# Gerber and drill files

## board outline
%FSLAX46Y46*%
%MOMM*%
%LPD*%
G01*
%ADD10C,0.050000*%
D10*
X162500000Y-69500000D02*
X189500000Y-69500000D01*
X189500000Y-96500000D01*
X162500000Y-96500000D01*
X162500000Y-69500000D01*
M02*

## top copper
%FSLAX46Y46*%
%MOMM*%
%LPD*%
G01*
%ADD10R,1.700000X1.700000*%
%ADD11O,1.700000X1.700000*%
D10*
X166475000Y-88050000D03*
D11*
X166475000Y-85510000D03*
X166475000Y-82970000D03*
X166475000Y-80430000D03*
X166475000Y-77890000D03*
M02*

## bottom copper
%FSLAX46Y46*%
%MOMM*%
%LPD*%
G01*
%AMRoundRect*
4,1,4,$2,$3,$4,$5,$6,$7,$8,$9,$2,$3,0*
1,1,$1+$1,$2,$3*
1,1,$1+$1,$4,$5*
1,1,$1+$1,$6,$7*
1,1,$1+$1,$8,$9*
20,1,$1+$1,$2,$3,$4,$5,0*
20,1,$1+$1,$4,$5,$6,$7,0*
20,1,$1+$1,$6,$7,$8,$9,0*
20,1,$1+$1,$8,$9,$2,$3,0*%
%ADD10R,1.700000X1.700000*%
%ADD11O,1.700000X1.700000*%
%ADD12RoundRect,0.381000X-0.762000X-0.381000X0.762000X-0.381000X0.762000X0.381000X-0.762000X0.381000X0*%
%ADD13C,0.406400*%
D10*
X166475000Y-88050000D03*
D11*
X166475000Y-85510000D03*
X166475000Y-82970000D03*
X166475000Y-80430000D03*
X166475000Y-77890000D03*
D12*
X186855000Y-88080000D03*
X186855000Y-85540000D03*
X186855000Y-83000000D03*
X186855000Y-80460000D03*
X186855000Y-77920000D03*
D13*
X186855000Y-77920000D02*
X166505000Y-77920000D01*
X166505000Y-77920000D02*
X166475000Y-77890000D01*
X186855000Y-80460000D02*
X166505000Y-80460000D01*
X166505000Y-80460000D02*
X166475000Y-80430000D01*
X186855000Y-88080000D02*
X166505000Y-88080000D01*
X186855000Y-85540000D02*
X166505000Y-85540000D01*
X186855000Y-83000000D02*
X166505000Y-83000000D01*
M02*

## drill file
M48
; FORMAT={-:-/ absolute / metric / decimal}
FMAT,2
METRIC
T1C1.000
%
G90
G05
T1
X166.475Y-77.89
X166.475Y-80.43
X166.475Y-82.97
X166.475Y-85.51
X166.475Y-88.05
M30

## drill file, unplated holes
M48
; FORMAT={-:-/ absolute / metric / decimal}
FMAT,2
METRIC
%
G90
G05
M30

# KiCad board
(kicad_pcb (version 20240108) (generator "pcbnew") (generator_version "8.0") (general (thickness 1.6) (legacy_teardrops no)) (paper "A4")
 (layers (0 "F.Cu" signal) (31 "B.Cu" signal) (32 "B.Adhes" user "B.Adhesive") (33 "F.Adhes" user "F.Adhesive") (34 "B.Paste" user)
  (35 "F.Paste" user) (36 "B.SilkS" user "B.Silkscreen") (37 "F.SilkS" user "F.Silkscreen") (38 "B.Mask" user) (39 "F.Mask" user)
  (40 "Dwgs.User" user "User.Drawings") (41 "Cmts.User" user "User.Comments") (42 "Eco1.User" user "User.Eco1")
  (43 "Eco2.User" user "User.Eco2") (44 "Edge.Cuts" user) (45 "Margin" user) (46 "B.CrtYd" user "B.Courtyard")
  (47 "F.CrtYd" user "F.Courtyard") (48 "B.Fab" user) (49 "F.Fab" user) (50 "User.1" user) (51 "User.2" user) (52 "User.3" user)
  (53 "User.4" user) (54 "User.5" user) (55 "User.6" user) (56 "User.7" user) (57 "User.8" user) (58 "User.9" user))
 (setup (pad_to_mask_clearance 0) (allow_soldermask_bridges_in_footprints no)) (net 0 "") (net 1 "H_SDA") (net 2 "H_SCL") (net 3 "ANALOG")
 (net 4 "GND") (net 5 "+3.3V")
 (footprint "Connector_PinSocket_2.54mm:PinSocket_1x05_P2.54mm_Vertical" (layer "F.Cu") (at 166.475 88.05 180)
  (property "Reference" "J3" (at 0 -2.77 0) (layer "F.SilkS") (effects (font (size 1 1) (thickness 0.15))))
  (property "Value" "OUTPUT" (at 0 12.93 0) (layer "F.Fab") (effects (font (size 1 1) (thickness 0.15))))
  (pad "1" thru_hole rect (at 0 0 180) (size 1.7 1.7) (drill 1) (layers "*.Cu" "*.Mask") (remove_unused_layers no) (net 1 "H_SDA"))
  (pad "2" thru_hole oval (at 0 2.54 180) (size 1.7 1.7) (drill 1) (layers "*.Cu" "*.Mask") (remove_unused_layers no) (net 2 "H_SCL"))
  (pad "3" thru_hole oval (at 0 5.08 180) (size 1.7 1.7) (drill 1) (layers "*.Cu" "*.Mask") (remove_unused_layers no) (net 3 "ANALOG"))
  (pad "4" thru_hole oval (at 0 7.62 180) (size 1.7 1.7) (drill 1) (layers "*.Cu" "*.Mask") (remove_unused_layers no) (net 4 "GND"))
  (pad "5" thru_hole oval (at 0 10.16 180) (size 1.7 1.7) (drill 1) (layers "*.Cu" "*.Mask") (remove_unused_layers no) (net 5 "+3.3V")))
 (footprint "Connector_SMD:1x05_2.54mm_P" (layer "B.Cu") (at 186.855 83 90)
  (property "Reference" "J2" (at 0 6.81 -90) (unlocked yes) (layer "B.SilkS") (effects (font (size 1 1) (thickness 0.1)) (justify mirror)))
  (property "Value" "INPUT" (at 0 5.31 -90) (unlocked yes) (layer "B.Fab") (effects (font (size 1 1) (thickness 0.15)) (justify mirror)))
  (pad "1" smd roundrect (at -5.08 0) (size 2.286 1.524) (layers "B.Cu" "B.Paste" "B.Mask") (roundrect_rratio 0.25) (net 1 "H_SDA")
   (thermal_bridge_angle 45))
  (pad "2" smd roundrect (at -2.54 0) (size 2.286 1.524) (layers "B.Cu" "B.Paste" "B.Mask") (roundrect_rratio 0.25) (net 2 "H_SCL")
   (thermal_bridge_angle 45))
  (pad "3" smd roundrect (at 0 0) (size 2.286 1.524) (layers "B.Cu" "B.Paste" "B.Mask") (roundrect_rratio 0.25) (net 3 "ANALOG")
   (thermal_bridge_angle 45))
  (pad "4" smd roundrect (at 2.54 0) (size 2.286 1.524) (layers "B.Cu" "B.Paste" "B.Mask") (roundrect_rratio 0.25) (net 4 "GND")
   (thermal_bridge_angle 45))
  (pad "5" smd roundrect (at 5.08 0) (size 2.286 1.524) (layers "B.Cu" "B.Paste" "B.Mask") (roundrect_rratio 0.25) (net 5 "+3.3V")
   (thermal_bridge_angle 45)))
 (gr_rect (start 162.5 69.5) (end 189.5 96.5) (stroke (width 0.05) (type default)) (fill none) (layer "Edge.Cuts"))
 (segment (start 166.505 77.92) (end 166.475 77.89) (width 0.4064) (layer "B.Cu") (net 5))
 (segment (start 186.855 77.92) (end 166.505 77.92) (width 0.4064) (layer "B.Cu") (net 5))
 (segment (start 186.855 80.46) (end 166.505 80.46) (width 0.4064) (layer "B.Cu") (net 4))
 (segment (start 166.505 80.46) (end 166.475 80.43) (width 0.4064) (layer "B.Cu") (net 4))
 (segment (start 186.855 83) (end 166.505 83) (width 0.4064) (layer "B.Cu") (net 3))
 (segment (start 186.855 88.08) (end 166.505 88.08) (width 0.4064) (layer "B.Cu") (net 1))
 (segment (start 186.855 85.54) (end 166.505 85.54) (width 0.4064) (layer "B.Cu") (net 2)))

